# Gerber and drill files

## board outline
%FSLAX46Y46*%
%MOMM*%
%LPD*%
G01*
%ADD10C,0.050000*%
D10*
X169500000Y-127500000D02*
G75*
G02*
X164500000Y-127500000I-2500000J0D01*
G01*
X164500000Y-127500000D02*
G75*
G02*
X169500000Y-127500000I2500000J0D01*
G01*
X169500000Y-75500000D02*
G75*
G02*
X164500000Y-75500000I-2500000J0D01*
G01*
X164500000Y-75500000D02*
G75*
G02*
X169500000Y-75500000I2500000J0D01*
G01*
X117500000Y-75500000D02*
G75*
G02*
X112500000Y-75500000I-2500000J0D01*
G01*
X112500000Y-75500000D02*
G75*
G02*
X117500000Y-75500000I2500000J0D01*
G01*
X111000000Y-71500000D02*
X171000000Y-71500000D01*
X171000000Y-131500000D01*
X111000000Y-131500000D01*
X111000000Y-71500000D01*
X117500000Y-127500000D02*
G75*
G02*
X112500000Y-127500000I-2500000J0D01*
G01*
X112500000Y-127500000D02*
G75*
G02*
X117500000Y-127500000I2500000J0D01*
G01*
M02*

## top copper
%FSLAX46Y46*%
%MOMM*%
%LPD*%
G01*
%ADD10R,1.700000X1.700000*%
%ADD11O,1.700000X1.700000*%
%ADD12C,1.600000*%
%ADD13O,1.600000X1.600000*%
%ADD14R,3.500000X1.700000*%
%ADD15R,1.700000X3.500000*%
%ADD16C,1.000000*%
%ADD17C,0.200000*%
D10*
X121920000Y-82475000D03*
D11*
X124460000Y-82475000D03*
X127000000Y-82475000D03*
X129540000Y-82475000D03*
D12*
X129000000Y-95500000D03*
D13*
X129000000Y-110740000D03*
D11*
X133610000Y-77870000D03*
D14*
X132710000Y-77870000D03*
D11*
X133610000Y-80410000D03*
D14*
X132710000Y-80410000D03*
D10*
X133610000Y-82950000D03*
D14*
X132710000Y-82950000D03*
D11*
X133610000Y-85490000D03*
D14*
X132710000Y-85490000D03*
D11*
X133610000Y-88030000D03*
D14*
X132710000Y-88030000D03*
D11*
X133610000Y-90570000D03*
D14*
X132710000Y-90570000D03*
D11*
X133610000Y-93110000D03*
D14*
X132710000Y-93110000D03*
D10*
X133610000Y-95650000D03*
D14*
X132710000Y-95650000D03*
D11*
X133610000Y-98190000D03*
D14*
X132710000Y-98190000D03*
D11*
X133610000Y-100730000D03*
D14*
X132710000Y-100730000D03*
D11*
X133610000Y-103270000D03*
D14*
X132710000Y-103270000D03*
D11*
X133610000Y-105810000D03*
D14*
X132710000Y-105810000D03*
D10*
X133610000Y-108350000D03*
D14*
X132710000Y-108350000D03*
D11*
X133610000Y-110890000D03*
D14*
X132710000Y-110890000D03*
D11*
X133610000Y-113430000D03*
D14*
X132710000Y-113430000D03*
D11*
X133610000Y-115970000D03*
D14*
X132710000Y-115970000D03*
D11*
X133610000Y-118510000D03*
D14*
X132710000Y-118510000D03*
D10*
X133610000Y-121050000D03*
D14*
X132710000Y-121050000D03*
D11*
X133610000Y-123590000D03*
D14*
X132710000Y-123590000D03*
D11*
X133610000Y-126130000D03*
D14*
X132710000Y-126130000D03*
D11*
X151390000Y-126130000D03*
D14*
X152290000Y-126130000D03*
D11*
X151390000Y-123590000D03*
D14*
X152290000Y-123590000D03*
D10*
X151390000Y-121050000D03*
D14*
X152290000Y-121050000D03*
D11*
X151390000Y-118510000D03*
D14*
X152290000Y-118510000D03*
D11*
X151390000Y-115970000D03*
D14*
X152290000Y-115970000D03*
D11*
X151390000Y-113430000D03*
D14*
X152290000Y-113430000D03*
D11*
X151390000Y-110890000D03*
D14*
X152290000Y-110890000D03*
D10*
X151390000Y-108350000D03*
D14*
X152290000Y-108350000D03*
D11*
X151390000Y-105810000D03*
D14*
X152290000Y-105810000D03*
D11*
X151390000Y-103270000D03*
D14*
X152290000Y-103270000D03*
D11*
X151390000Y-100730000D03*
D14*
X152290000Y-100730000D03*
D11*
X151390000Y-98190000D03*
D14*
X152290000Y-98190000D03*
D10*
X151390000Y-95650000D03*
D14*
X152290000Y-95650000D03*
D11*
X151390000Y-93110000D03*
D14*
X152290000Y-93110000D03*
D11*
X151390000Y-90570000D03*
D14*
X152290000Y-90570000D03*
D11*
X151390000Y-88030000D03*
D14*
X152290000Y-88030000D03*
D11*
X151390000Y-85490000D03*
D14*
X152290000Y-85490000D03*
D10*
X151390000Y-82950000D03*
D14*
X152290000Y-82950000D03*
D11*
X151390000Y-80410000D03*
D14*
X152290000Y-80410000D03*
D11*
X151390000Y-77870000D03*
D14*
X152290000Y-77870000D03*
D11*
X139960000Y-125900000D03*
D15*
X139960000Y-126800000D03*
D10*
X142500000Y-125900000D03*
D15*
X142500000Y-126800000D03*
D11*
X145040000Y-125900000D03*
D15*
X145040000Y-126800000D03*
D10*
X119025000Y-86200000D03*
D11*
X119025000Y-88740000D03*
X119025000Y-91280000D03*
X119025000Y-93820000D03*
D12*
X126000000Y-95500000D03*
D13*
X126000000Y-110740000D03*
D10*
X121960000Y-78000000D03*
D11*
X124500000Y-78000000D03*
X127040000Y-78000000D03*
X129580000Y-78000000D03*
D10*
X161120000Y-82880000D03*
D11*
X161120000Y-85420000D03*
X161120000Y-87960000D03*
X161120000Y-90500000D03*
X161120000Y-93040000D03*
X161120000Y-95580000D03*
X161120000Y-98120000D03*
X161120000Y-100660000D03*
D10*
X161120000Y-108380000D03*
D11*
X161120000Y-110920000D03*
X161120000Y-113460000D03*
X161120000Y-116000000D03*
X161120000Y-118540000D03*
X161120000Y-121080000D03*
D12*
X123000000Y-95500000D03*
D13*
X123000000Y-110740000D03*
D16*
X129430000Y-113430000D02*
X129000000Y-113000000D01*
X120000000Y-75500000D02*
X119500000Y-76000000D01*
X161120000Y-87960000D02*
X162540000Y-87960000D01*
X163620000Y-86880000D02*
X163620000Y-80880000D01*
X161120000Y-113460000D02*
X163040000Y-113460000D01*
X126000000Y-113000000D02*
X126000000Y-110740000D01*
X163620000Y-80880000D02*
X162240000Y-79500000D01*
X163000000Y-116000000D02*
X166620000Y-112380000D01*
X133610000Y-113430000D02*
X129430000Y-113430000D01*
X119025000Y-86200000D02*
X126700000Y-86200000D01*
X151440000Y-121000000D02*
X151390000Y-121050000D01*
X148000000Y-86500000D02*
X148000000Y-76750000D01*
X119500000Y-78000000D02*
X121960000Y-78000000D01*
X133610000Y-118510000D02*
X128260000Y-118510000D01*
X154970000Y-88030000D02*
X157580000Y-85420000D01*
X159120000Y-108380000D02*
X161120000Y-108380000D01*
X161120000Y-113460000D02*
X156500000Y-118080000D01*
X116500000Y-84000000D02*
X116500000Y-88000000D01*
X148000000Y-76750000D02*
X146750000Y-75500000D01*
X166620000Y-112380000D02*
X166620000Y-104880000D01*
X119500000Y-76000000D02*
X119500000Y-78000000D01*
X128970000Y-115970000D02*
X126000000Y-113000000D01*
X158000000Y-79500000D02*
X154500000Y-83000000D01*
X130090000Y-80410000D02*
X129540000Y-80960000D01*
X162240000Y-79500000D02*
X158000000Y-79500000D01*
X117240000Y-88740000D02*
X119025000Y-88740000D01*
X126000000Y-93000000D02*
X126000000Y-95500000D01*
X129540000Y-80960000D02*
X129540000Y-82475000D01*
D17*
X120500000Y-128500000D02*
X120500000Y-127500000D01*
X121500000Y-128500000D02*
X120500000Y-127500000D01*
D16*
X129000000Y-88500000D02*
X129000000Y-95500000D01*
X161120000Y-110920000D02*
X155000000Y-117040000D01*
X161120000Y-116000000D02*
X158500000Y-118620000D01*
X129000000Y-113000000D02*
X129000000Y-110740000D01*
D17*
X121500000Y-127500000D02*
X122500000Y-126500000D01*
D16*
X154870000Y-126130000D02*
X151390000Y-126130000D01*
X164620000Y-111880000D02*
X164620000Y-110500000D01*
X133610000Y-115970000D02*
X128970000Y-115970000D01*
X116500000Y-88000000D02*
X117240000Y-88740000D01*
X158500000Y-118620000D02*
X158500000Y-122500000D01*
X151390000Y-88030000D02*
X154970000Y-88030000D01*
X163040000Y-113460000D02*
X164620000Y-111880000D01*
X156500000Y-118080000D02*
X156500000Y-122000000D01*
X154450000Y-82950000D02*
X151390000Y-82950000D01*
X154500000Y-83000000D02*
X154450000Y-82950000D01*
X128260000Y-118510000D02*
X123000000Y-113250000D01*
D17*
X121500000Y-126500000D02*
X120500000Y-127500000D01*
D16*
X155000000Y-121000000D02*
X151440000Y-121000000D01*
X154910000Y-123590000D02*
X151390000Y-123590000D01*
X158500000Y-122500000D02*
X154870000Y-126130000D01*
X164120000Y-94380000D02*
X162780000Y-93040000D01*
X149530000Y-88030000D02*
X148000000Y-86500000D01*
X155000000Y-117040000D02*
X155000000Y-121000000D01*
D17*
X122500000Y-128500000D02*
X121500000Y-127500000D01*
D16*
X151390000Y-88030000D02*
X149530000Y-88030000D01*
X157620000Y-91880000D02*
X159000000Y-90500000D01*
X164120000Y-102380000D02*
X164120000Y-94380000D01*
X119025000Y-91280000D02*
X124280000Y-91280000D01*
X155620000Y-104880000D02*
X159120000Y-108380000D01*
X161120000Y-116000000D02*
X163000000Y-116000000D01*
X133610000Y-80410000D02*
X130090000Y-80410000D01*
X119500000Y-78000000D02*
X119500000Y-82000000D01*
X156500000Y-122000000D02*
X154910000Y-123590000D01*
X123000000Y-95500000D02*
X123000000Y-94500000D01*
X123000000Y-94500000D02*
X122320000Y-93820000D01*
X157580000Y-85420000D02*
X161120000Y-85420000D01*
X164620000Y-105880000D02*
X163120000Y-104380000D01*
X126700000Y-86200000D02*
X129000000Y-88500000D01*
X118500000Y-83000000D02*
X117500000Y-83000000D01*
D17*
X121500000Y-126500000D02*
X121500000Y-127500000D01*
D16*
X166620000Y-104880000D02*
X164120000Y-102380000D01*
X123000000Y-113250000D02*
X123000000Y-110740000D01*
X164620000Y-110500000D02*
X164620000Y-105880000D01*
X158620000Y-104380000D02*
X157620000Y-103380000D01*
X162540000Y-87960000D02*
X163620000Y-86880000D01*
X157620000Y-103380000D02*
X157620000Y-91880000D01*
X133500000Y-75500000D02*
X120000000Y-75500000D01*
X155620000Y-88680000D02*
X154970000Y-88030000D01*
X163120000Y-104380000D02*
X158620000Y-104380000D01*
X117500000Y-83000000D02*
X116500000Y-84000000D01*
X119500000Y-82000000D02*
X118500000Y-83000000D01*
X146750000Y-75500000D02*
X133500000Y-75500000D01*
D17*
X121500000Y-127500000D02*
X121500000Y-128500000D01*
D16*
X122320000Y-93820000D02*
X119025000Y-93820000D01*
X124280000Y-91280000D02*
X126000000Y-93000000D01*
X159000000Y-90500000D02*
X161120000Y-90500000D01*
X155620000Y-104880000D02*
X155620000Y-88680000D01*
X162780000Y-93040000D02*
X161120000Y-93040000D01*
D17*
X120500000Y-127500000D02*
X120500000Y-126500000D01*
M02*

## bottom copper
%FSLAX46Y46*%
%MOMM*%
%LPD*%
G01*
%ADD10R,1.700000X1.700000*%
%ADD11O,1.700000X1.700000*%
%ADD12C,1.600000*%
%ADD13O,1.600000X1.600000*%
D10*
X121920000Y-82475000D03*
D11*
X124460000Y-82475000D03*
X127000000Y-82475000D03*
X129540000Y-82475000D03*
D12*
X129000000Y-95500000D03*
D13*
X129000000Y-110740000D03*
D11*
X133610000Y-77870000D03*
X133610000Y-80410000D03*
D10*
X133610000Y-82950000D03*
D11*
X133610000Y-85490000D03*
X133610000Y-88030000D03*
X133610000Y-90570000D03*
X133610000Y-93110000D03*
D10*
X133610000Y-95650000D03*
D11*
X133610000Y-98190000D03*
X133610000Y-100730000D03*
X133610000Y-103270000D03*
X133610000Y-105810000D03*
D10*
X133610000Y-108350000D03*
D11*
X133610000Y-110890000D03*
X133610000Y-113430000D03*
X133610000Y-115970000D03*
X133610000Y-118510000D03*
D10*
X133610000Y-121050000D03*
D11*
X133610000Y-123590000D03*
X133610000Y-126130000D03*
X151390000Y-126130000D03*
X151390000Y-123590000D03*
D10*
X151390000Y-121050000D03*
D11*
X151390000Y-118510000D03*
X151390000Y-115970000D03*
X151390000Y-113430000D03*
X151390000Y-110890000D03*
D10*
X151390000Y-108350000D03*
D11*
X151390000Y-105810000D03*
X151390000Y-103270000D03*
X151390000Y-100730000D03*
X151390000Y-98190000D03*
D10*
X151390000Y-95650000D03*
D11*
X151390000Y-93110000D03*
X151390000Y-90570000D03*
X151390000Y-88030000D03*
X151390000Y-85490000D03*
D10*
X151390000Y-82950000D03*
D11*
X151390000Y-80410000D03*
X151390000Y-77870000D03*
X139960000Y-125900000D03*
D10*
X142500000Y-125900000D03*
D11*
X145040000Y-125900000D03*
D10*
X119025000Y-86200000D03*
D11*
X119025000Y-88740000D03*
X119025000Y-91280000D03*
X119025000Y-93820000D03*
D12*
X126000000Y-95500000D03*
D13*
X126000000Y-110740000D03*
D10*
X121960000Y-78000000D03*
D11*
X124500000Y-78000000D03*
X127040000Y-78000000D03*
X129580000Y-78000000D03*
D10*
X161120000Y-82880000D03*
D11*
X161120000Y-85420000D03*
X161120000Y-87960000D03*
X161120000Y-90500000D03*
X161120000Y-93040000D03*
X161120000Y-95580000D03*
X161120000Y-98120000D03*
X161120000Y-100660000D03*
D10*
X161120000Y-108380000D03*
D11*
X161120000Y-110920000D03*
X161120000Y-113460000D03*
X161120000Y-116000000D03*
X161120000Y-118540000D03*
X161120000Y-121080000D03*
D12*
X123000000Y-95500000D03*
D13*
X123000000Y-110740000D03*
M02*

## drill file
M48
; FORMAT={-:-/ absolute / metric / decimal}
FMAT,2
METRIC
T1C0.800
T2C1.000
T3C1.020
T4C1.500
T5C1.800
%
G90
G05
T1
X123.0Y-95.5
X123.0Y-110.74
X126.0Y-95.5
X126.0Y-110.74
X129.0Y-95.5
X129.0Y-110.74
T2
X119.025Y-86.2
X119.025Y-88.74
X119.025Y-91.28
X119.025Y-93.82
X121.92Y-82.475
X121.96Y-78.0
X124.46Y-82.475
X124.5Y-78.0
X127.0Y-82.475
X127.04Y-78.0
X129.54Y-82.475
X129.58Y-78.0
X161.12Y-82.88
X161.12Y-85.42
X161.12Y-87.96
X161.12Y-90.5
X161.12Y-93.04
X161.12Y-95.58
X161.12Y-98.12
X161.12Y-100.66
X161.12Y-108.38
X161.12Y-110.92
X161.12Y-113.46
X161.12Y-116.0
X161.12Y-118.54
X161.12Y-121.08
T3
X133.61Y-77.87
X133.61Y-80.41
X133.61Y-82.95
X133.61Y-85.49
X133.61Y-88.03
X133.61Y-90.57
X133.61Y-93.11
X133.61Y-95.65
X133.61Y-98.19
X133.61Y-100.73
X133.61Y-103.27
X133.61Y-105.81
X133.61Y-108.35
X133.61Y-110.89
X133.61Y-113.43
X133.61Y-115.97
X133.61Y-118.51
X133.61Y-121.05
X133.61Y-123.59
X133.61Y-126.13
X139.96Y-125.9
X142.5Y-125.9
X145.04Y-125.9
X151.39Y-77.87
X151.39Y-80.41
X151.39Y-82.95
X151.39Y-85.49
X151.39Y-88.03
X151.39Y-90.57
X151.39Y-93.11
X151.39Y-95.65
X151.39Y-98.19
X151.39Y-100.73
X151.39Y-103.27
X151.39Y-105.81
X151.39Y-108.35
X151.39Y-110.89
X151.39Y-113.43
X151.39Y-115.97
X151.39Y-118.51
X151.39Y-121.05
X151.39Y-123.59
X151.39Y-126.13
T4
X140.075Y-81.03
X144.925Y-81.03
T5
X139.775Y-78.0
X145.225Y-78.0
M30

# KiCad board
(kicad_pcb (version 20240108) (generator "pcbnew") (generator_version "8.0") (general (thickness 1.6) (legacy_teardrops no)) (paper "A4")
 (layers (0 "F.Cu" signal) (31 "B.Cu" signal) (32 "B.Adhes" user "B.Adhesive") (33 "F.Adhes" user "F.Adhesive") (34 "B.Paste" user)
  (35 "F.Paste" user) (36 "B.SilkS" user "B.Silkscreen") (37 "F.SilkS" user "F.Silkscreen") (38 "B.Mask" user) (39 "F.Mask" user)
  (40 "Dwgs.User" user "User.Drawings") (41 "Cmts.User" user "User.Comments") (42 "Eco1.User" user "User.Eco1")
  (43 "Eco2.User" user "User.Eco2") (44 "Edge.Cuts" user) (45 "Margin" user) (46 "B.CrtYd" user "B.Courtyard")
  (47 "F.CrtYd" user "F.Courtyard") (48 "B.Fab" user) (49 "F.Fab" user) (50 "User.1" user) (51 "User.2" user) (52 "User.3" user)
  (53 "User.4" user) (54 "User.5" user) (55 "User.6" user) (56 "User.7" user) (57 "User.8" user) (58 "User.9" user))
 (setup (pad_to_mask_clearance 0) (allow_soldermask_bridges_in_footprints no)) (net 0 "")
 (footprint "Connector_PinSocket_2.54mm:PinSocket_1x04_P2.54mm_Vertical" (layer "F.Cu") (at 121.92 82.475 90)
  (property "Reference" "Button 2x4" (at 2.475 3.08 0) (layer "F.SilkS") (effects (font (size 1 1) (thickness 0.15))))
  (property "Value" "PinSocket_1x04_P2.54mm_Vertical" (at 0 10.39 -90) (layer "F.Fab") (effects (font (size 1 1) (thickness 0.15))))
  (pad "1" thru_hole rect (at 0 0 90) (size 1.7 1.7) (drill 1) (layers "*.Cu" "*.Mask") (remove_unused_layers no))
  (pad "2" thru_hole oval (at 0 2.54 90) (size 1.7 1.7) (drill 1) (layers "*.Cu" "*.Mask") (remove_unused_layers no))
  (pad "3" thru_hole oval (at 0 5.08 90) (size 1.7 1.7) (drill 1) (layers "*.Cu" "*.Mask") (remove_unused_layers no))
  (pad "4" thru_hole oval (at 0 7.62 90) (size 1.7 1.7) (drill 1) (layers "*.Cu" "*.Mask") (remove_unused_layers no)))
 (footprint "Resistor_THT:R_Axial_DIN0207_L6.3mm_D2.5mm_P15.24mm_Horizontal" (layer "F.Cu") (at 129 95.5 -90)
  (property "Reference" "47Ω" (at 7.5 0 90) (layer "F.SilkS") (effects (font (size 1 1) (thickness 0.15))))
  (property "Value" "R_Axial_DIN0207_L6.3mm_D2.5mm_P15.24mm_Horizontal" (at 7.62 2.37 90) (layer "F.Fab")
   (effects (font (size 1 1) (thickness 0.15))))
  (pad "1" thru_hole circle (at 0 0 270) (size 1.6 1.6) (drill 0.8) (layers "*.Cu" "*.Mask") (remove_unused_layers no))
  (pad "2" thru_hole oval (at 15.24 0 270) (size 1.6 1.6) (drill 0.8) (layers "*.Cu" "*.Mask") (remove_unused_layers no)))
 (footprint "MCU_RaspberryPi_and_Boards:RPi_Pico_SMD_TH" (layer "F.Cu") (at 142.5 102)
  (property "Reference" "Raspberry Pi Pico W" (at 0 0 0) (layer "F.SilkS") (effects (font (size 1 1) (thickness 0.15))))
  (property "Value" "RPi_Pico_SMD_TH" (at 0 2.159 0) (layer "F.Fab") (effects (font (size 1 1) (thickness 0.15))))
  (pad "" np_thru_hole oval (at -2.725 -24) (size 1.8 1.8) (drill 1.8) (layers "*.Cu" "*.Mask"))
  (pad "" np_thru_hole oval (at -2.425 -20.97) (size 1.5 1.5) (drill 1.5) (layers "*.Cu" "*.Mask"))
  (pad "" np_thru_hole oval (at 2.425 -20.97) (size 1.5 1.5) (drill 1.5) (layers "*.Cu" "*.Mask"))
  (pad "" np_thru_hole oval (at 2.725 -24) (size 1.8 1.8) (drill 1.8) (layers "*.Cu" "*.Mask"))
  (pad "1" thru_hole oval (at -8.89 -24.13) (size 1.7 1.7) (drill 1.02) (layers "*.Cu" "*.Mask") (remove_unused_layers no))
  (pad "1" smd rect (at -8.89 -24.13) (size 3.5 1.7) (drill (offset -0.9 0)) (layers "F.Cu" "F.Mask"))
  (pad "2" thru_hole oval (at -8.89 -21.59) (size 1.7 1.7) (drill 1.02) (layers "*.Cu" "*.Mask") (remove_unused_layers no))
  (pad "2" smd rect (at -8.89 -21.59) (size 3.5 1.7) (drill (offset -0.9 0)) (layers "F.Cu" "F.Mask"))
  (pad "3" thru_hole rect (at -8.89 -19.05) (size 1.7 1.7) (drill 1.02) (layers "*.Cu" "*.Mask") (remove_unused_layers no))
  (pad "3" smd rect (at -8.89 -19.05) (size 3.5 1.7) (drill (offset -0.9 0)) (layers "F.Cu" "F.Mask"))
  (pad "4" thru_hole oval (at -8.89 -16.51) (size 1.7 1.7) (drill 1.02) (layers "*.Cu" "*.Mask") (remove_unused_layers no))
  (pad "4" smd rect (at -8.89 -16.51) (size 3.5 1.7) (drill (offset -0.9 0)) (layers "F.Cu" "F.Mask"))
  (pad "5" thru_hole oval (at -8.89 -13.97) (size 1.7 1.7) (drill 1.02) (layers "*.Cu" "*.Mask") (remove_unused_layers no))
  (pad "5" smd rect (at -8.89 -13.97) (size 3.5 1.7) (drill (offset -0.9 0)) (layers "F.Cu" "F.Mask"))
  (pad "6" thru_hole oval (at -8.89 -11.43) (size 1.7 1.7) (drill 1.02) (layers "*.Cu" "*.Mask") (remove_unused_layers no))
  (pad "6" smd rect (at -8.89 -11.43) (size 3.5 1.7) (drill (offset -0.9 0)) (layers "F.Cu" "F.Mask"))
  (pad "7" thru_hole oval (at -8.89 -8.89) (size 1.7 1.7) (drill 1.02) (layers "*.Cu" "*.Mask") (remove_unused_layers no))
  (pad "7" smd rect (at -8.89 -8.89) (size 3.5 1.7) (drill (offset -0.9 0)) (layers "F.Cu" "F.Mask"))
  (pad "8" thru_hole rect (at -8.89 -6.35) (size 1.7 1.7) (drill 1.02) (layers "*.Cu" "*.Mask") (remove_unused_layers no))
  (pad "8" smd rect (at -8.89 -6.35) (size 3.5 1.7) (drill (offset -0.9 0)) (layers "F.Cu" "F.Mask"))
  (pad "9" thru_hole oval (at -8.89 -3.81) (size 1.7 1.7) (drill 1.02) (layers "*.Cu" "*.Mask") (remove_unused_layers no))
  (pad "9" smd rect (at -8.89 -3.81) (size 3.5 1.7) (drill (offset -0.9 0)) (layers "F.Cu" "F.Mask"))
  (pad "10" thru_hole oval (at -8.89 -1.27) (size 1.7 1.7) (drill 1.02) (layers "*.Cu" "*.Mask") (remove_unused_layers no))
  (pad "10" smd rect (at -8.89 -1.27) (size 3.5 1.7) (drill (offset -0.9 0)) (layers "F.Cu" "F.Mask"))
  (pad "11" thru_hole oval (at -8.89 1.27) (size 1.7 1.7) (drill 1.02) (layers "*.Cu" "*.Mask") (remove_unused_layers no))
  (pad "11" smd rect (at -8.89 1.27) (size 3.5 1.7) (drill (offset -0.9 0)) (layers "F.Cu" "F.Mask"))
  (pad "12" thru_hole oval (at -8.89 3.81) (size 1.7 1.7) (drill 1.02) (layers "*.Cu" "*.Mask") (remove_unused_layers no))
  (pad "12" smd rect (at -8.89 3.81) (size 3.5 1.7) (drill (offset -0.9 0)) (layers "F.Cu" "F.Mask"))
  (pad "13" thru_hole rect (at -8.89 6.35) (size 1.7 1.7) (drill 1.02) (layers "*.Cu" "*.Mask") (remove_unused_layers no))
  (pad "13" smd rect (at -8.89 6.35) (size 3.5 1.7) (drill (offset -0.9 0)) (layers "F.Cu" "F.Mask"))
  (pad "14" thru_hole oval (at -8.89 8.89) (size 1.7 1.7) (drill 1.02) (layers "*.Cu" "*.Mask") (remove_unused_layers no))
  (pad "14" smd rect (at -8.89 8.89) (size 3.5 1.7) (drill (offset -0.9 0)) (layers "F.Cu" "F.Mask"))
  (pad "15" thru_hole oval (at -8.89 11.43) (size 1.7 1.7) (drill 1.02) (layers "*.Cu" "*.Mask") (remove_unused_layers no))
  (pad "15" smd rect (at -8.89 11.43) (size 3.5 1.7) (drill (offset -0.9 0)) (layers "F.Cu" "F.Mask"))
  (pad "16" thru_hole oval (at -8.89 13.97) (size 1.7 1.7) (drill 1.02) (layers "*.Cu" "*.Mask") (remove_unused_layers no))
  (pad "16" smd rect (at -8.89 13.97) (size 3.5 1.7) (drill (offset -0.9 0)) (layers "F.Cu" "F.Mask"))
  (pad "17" thru_hole oval (at -8.89 16.51) (size 1.7 1.7) (drill 1.02) (layers "*.Cu" "*.Mask") (remove_unused_layers no))
  (pad "17" smd rect (at -8.89 16.51) (size 3.5 1.7) (drill (offset -0.9 0)) (layers "F.Cu" "F.Mask"))
  (pad "18" thru_hole rect (at -8.89 19.05) (size 1.7 1.7) (drill 1.02) (layers "*.Cu" "*.Mask") (remove_unused_layers no))
  (pad "18" smd rect (at -8.89 19.05) (size 3.5 1.7) (drill (offset -0.9 0)) (layers "F.Cu" "F.Mask"))
  (pad "19" thru_hole oval (at -8.89 21.59) (size 1.7 1.7) (drill 1.02) (layers "*.Cu" "*.Mask") (remove_unused_layers no))
  (pad "19" smd rect (at -8.89 21.59) (size 3.5 1.7) (drill (offset -0.9 0)) (layers "F.Cu" "F.Mask"))
  (pad "20" thru_hole oval (at -8.89 24.13) (size 1.7 1.7) (drill 1.02) (layers "*.Cu" "*.Mask") (remove_unused_layers no))
  (pad "20" smd rect (at -8.89 24.13) (size 3.5 1.7) (drill (offset -0.9 0)) (layers "F.Cu" "F.Mask"))
  (pad "21" thru_hole oval (at 8.89 24.13) (size 1.7 1.7) (drill 1.02) (layers "*.Cu" "*.Mask") (remove_unused_layers no))
  (pad "21" smd rect (at 8.89 24.13) (size 3.5 1.7) (drill (offset 0.9 0)) (layers "F.Cu" "F.Mask"))
  (pad "22" thru_hole oval (at 8.89 21.59) (size 1.7 1.7) (drill 1.02) (layers "*.Cu" "*.Mask") (remove_unused_layers no))
  (pad "22" smd rect (at 8.89 21.59) (size 3.5 1.7) (drill (offset 0.9 0)) (layers "F.Cu" "F.Mask"))
  (pad "23" thru_hole rect (at 8.89 19.05) (size 1.7 1.7) (drill 1.02) (layers "*.Cu" "*.Mask") (remove_unused_layers no))
  (pad "23" smd rect (at 8.89 19.05) (size 3.5 1.7) (drill (offset 0.9 0)) (layers "F.Cu" "F.Mask"))
  (pad "24" thru_hole oval (at 8.89 16.51) (size 1.7 1.7) (drill 1.02) (layers "*.Cu" "*.Mask") (remove_unused_layers no))
  (pad "24" smd rect (at 8.89 16.51) (size 3.5 1.7) (drill (offset 0.9 0)) (layers "F.Cu" "F.Mask"))
  (pad "25" thru_hole oval (at 8.89 13.97) (size 1.7 1.7) (drill 1.02) (layers "*.Cu" "*.Mask") (remove_unused_layers no))
  (pad "25" smd rect (at 8.89 13.97) (size 3.5 1.7) (drill (offset 0.9 0)) (layers "F.Cu" "F.Mask"))
  (pad "26" thru_hole oval (at 8.89 11.43) (size 1.7 1.7) (drill 1.02) (layers "*.Cu" "*.Mask") (remove_unused_layers no))
  (pad "26" smd rect (at 8.89 11.43) (size 3.5 1.7) (drill (offset 0.9 0)) (layers "F.Cu" "F.Mask"))
  (pad "27" thru_hole oval (at 8.89 8.89) (size 1.7 1.7) (drill 1.02) (layers "*.Cu" "*.Mask") (remove_unused_layers no))
  (pad "27" smd rect (at 8.89 8.89) (size 3.5 1.7) (drill (offset 0.9 0)) (layers "F.Cu" "F.Mask"))
  (pad "28" thru_hole rect (at 8.89 6.35) (size 1.7 1.7) (drill 1.02) (layers "*.Cu" "*.Mask") (remove_unused_layers no))
  (pad "28" smd rect (at 8.89 6.35) (size 3.5 1.7) (drill (offset 0.9 0)) (layers "F.Cu" "F.Mask"))
  (pad "29" thru_hole oval (at 8.89 3.81) (size 1.7 1.7) (drill 1.02) (layers "*.Cu" "*.Mask") (remove_unused_layers no))
  (pad "29" smd rect (at 8.89 3.81) (size 3.5 1.7) (drill (offset 0.9 0)) (layers "F.Cu" "F.Mask"))
  (pad "30" thru_hole oval (at 8.89 1.27) (size 1.7 1.7) (drill 1.02) (layers "*.Cu" "*.Mask") (remove_unused_layers no))
  (pad "30" smd rect (at 8.89 1.27) (size 3.5 1.7) (drill (offset 0.9 0)) (layers "F.Cu" "F.Mask"))
  (pad "31" thru_hole oval (at 8.89 -1.27) (size 1.7 1.7) (drill 1.02) (layers "*.Cu" "*.Mask") (remove_unused_layers no))
  (pad "31" smd rect (at 8.89 -1.27) (size 3.5 1.7) (drill (offset 0.9 0)) (layers "F.Cu" "F.Mask"))
  (pad "32" thru_hole oval (at 8.89 -3.81) (size 1.7 1.7) (drill 1.02) (layers "*.Cu" "*.Mask") (remove_unused_layers no))
  (pad "32" smd rect (at 8.89 -3.81) (size 3.5 1.7) (drill (offset 0.9 0)) (layers "F.Cu" "F.Mask"))
  (pad "33" thru_hole rect (at 8.89 -6.35) (size 1.7 1.7) (drill 1.02) (layers "*.Cu" "*.Mask") (remove_unused_layers no))
  (pad "33" smd rect (at 8.89 -6.35) (size 3.5 1.7) (drill (offset 0.9 0)) (layers "F.Cu" "F.Mask"))
  (pad "34" thru_hole oval (at 8.89 -8.89) (size 1.7 1.7) (drill 1.02) (layers "*.Cu" "*.Mask") (remove_unused_layers no))
  (pad "34" smd rect (at 8.89 -8.89) (size 3.5 1.7) (drill (offset 0.9 0)) (layers "F.Cu" "F.Mask"))
  (pad "35" thru_hole oval (at 8.89 -11.43) (size 1.7 1.7) (drill 1.02) (layers "*.Cu" "*.Mask") (remove_unused_layers no))
  (pad "35" smd rect (at 8.89 -11.43) (size 3.5 1.7) (drill (offset 0.9 0)) (layers "F.Cu" "F.Mask"))
  (pad "36" thru_hole oval (at 8.89 -13.97) (size 1.7 1.7) (drill 1.02) (layers "*.Cu" "*.Mask") (remove_unused_layers no))
  (pad "36" smd rect (at 8.89 -13.97) (size 3.5 1.7) (drill (offset 0.9 0)) (layers "F.Cu" "F.Mask"))
  (pad "37" thru_hole oval (at 8.89 -16.51) (size 1.7 1.7) (drill 1.02) (layers "*.Cu" "*.Mask") (remove_unused_layers no))
  (pad "37" smd rect (at 8.89 -16.51) (size 3.5 1.7) (drill (offset 0.9 0)) (layers "F.Cu" "F.Mask"))
  (pad "38" thru_hole rect (at 8.89 -19.05) (size 1.7 1.7) (drill 1.02) (layers "*.Cu" "*.Mask") (remove_unused_layers no))
  (pad "38" smd rect (at 8.89 -19.05) (size 3.5 1.7) (drill (offset 0.9 0)) (layers "F.Cu" "F.Mask"))
  (pad "39" thru_hole oval (at 8.89 -21.59) (size 1.7 1.7) (drill 1.02) (layers "*.Cu" "*.Mask") (remove_unused_layers no))
  (pad "39" smd rect (at 8.89 -21.59) (size 3.5 1.7) (drill (offset 0.9 0)) (layers "F.Cu" "F.Mask"))
  (pad "40" thru_hole oval (at 8.89 -24.13) (size 1.7 1.7) (drill 1.02) (layers "*.Cu" "*.Mask") (remove_unused_layers no))
  (pad "40" smd rect (at 8.89 -24.13) (size 3.5 1.7) (drill (offset 0.9 0)) (layers "F.Cu" "F.Mask"))
  (pad "41" thru_hole oval (at -2.54 23.9) (size 1.7 1.7) (drill 1.02) (layers "*.Cu" "*.Mask") (remove_unused_layers no))
  (pad "41" smd rect (at -2.54 23.9 90) (size 3.5 1.7) (drill (offset -0.9 0)) (layers "F.Cu" "F.Mask"))
  (pad "42" thru_hole rect (at 0 23.9) (size 1.7 1.7) (drill 1.02) (layers "*.Cu" "*.Mask") (remove_unused_layers no))
  (pad "42" smd rect (at 0 23.9 90) (size 3.5 1.7) (drill (offset -0.9 0)) (layers "F.Cu" "F.Mask"))
  (pad "43" thru_hole oval (at 2.54 23.9) (size 1.7 1.7) (drill 1.02) (layers "*.Cu" "*.Mask") (remove_unused_layers no))
  (pad "43" smd rect (at 2.54 23.9 90) (size 3.5 1.7) (drill (offset -0.9 0)) (layers "F.Cu" "F.Mask")))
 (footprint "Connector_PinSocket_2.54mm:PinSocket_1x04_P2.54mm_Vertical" (layer "F.Cu") (at 119.025 86.2)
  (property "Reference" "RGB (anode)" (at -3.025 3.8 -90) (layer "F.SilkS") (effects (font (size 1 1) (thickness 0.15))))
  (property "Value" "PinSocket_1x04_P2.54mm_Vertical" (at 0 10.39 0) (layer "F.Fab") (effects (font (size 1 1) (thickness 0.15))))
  (pad "1" thru_hole rect (at 0 0) (size 1.7 1.7) (drill 1) (layers "*.Cu" "*.Mask") (remove_unused_layers no))
  (pad "2" thru_hole oval (at 0 2.54) (size 1.7 1.7) (drill 1) (layers "*.Cu" "*.Mask") (remove_unused_layers no))
  (pad "3" thru_hole oval (at 0 5.08) (size 1.7 1.7) (drill 1) (layers "*.Cu" "*.Mask") (remove_unused_layers no))
  (pad "4" thru_hole oval (at 0 7.62) (size 1.7 1.7) (drill 1) (layers "*.Cu" "*.Mask") (remove_unused_layers no)))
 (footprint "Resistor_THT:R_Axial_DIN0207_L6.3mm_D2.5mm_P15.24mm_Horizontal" (layer "F.Cu") (at 126 95.5 -90)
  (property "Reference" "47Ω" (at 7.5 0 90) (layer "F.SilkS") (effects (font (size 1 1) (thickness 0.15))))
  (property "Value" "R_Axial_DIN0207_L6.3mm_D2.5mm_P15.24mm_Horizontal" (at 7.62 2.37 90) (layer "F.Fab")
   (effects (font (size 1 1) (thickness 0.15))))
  (pad "1" thru_hole circle (at 0 0 270) (size 1.6 1.6) (drill 0.8) (layers "*.Cu" "*.Mask") (remove_unused_layers no))
  (pad "2" thru_hole oval (at 15.24 0 270) (size 1.6 1.6) (drill 0.8) (layers "*.Cu" "*.Mask") (remove_unused_layers no)))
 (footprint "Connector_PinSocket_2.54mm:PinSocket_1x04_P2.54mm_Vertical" (layer "F.Cu") (at 121.96 78 90)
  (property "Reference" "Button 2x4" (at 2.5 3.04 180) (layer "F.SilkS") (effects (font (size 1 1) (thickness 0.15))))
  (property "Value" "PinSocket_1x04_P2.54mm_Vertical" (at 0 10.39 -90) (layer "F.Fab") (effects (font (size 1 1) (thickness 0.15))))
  (pad "1" thru_hole rect (at 0 0 90) (size 1.7 1.7) (drill 1) (layers "*.Cu" "*.Mask") (remove_unused_layers no))
  (pad "2" thru_hole oval (at 0 2.54 90) (size 1.7 1.7) (drill 1) (layers "*.Cu" "*.Mask") (remove_unused_layers no))
  (pad "3" thru_hole oval (at 0 5.08 90) (size 1.7 1.7) (drill 1) (layers "*.Cu" "*.Mask") (remove_unused_layers no))
  (pad "4" thru_hole oval (at 0 7.62 90) (size 1.7 1.7) (drill 1) (layers "*.Cu" "*.Mask") (remove_unused_layers no)))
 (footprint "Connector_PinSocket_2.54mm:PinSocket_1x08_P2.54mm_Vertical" (layer "F.Cu") (at 161.12 82.88)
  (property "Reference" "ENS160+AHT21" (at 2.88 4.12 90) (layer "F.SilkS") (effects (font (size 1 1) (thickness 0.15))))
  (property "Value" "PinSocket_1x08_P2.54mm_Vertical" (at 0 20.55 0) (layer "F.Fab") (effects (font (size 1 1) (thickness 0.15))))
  (pad "1" thru_hole rect (at 0 0) (size 1.7 1.7) (drill 1) (layers "*.Cu" "*.Mask") (remove_unused_layers no))
  (pad "2" thru_hole oval (at 0 2.54) (size 1.7 1.7) (drill 1) (layers "*.Cu" "*.Mask") (remove_unused_layers no))
  (pad "3" thru_hole oval (at 0 5.08) (size 1.7 1.7) (drill 1) (layers "*.Cu" "*.Mask") (remove_unused_layers no))
  (pad "4" thru_hole oval (at 0 7.62) (size 1.7 1.7) (drill 1) (layers "*.Cu" "*.Mask") (remove_unused_layers no))
  (pad "5" thru_hole oval (at 0 10.16) (size 1.7 1.7) (drill 1) (layers "*.Cu" "*.Mask") (remove_unused_layers no))
  (pad "6" thru_hole oval (at 0 12.7) (size 1.7 1.7) (drill 1) (layers "*.Cu" "*.Mask") (remove_unused_layers no))
  (pad "7" thru_hole oval (at 0 15.24) (size 1.7 1.7) (drill 1) (layers "*.Cu" "*.Mask") (remove_unused_layers no))
  (pad "8" thru_hole oval (at 0 17.78) (size 1.7 1.7) (drill 1) (layers "*.Cu" "*.Mask") (remove_unused_layers no)))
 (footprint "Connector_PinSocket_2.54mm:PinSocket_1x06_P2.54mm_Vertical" (layer "F.Cu") (at 161.12 108.38)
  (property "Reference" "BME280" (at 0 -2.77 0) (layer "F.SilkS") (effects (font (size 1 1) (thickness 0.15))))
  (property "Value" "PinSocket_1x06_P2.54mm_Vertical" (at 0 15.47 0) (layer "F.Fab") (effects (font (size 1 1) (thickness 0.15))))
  (pad "1" thru_hole rect (at 0 0) (size 1.7 1.7) (drill 1) (layers "*.Cu" "*.Mask") (remove_unused_layers no))
  (pad "2" thru_hole oval (at 0 2.54) (size 1.7 1.7) (drill 1) (layers "*.Cu" "*.Mask") (remove_unused_layers no))
  (pad "3" thru_hole oval (at 0 5.08) (size 1.7 1.7) (drill 1) (layers "*.Cu" "*.Mask") (remove_unused_layers no))
  (pad "4" thru_hole oval (at 0 7.62) (size 1.7 1.7) (drill 1) (layers "*.Cu" "*.Mask") (remove_unused_layers no))
  (pad "5" thru_hole oval (at 0 10.16) (size 1.7 1.7) (drill 1) (layers "*.Cu" "*.Mask") (remove_unused_layers no))
  (pad "6" thru_hole oval (at 0 12.7) (size 1.7 1.7) (drill 1) (layers "*.Cu" "*.Mask") (remove_unused_layers no)))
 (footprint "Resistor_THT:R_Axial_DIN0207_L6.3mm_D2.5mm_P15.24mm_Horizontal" (layer "F.Cu") (at 123 95.5 -90)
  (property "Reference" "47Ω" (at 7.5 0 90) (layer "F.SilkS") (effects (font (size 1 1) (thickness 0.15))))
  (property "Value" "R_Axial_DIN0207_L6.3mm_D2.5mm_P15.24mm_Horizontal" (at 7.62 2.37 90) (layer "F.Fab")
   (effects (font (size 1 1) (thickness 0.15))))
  (pad "1" thru_hole circle (at 0 0 270) (size 1.6 1.6) (drill 0.8) (layers "*.Cu" "*.Mask") (remove_unused_layers no))
  (pad "2" thru_hole oval (at 15.24 0 270) (size 1.6 1.6) (drill 0.8) (layers "*.Cu" "*.Mask") (remove_unused_layers no)))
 (gr_circle (center 167 127.5) (end 165 126) (stroke (width 0.05) (type default)) (fill none) (layer "Edge.Cuts"))
 (gr_circle (center 167 75.5) (end 165.5 77.5) (stroke (width 0.05) (type default)) (fill none) (layer "Edge.Cuts"))
 (gr_circle (center 115 75.5) (end 113.5 73.5) (stroke (width 0.05) (type default)) (fill none) (layer "Edge.Cuts"))
 (gr_rect (start 111 71.5) (end 171 131.5) (stroke (width 0.05) (type default)) (fill none) (layer "Edge.Cuts"))
 (gr_circle (center 115 127.5) (end 117 126) (stroke (width 0.05) (type default)) (fill none) (layer "Edge.Cuts"))
 (segment (start 129.43 113.43) (end 129 113) (width 1) (layer "F.Cu") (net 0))
 (segment (start 120 75.5) (end 119.5 76) (width 1) (layer "F.Cu") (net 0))
 (segment (start 161.12 87.96) (end 162.54 87.96) (width 1) (layer "F.Cu") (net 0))
 (segment (start 163.62 86.88) (end 163.62 80.88) (width 1) (layer "F.Cu") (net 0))
 (segment (start 161.12 113.46) (end 163.04 113.46) (width 1) (layer "F.Cu") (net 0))
 (segment (start 126 113) (end 126 110.74) (width 1) (layer "F.Cu") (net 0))
 (segment (start 163.62 80.88) (end 162.24 79.5) (width 1) (layer "F.Cu") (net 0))
 (segment (start 163 116) (end 166.62 112.38) (width 1) (layer "F.Cu") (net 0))
 (segment (start 133.61 113.43) (end 129.43 113.43) (width 1) (layer "F.Cu") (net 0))
 (segment (start 119.025 86.2) (end 126.7 86.2) (width 1) (layer "F.Cu") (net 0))
 (segment (start 151.44 121) (end 151.39 121.05) (width 1) (layer "F.Cu") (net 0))
 (segment (start 148 86.5) (end 148 76.75) (width 1) (layer "F.Cu") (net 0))
 (segment (start 119.5 78) (end 121.96 78) (width 1) (layer "F.Cu") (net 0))
 (segment (start 133.61 118.51) (end 128.26 118.51) (width 1) (layer "F.Cu") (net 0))
 (segment (start 154.97 88.03) (end 157.58 85.42) (width 1) (layer "F.Cu") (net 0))
 (segment (start 159.12 108.38) (end 161.12 108.38) (width 1) (layer "F.Cu") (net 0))
 (segment (start 161.12 113.46) (end 156.5 118.08) (width 1) (layer "F.Cu") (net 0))
 (segment (start 116.5 84) (end 116.5 88) (width 1) (layer "F.Cu") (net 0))
 (segment (start 148 76.75) (end 146.75 75.5) (width 1) (layer "F.Cu") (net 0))
 (segment (start 166.62 112.38) (end 166.62 104.88) (width 1) (layer "F.Cu") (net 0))
 (segment (start 119.5 76) (end 119.5 78) (width 1) (layer "F.Cu") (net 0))
 (segment (start 128.97 115.97) (end 126 113) (width 1) (layer "F.Cu") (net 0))
 (segment (start 158 79.5) (end 154.5 83) (width 1) (layer "F.Cu") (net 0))
 (segment (start 130.09 80.41) (end 129.54 80.96) (width 1) (layer "F.Cu") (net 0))
 (segment (start 162.24 79.5) (end 158 79.5) (width 1) (layer "F.Cu") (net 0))
 (segment (start 117.24 88.74) (end 119.025 88.74) (width 1) (layer "F.Cu") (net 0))
 (segment (start 126 93) (end 126 95.5) (width 1) (layer "F.Cu") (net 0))
 (segment (start 129.54 80.96) (end 129.54 82.475) (width 1) (layer "F.Cu") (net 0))
 (segment (start 120.5 128.5) (end 120.5 127.5) (width 0.2) (layer "F.Cu") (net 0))
 (segment (start 121.5 128.5) (end 120.5 127.5) (width 0.2) (layer "F.Cu") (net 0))
 (segment (start 129 88.5) (end 129 95.5) (width 1) (layer "F.Cu") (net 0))
 (segment (start 161.12 110.92) (end 155 117.04) (width 1) (layer "F.Cu") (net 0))
 (segment (start 161.12 116) (end 158.5 118.62) (width 1) (layer "F.Cu") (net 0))
 (segment (start 129 113) (end 129 110.74) (width 1) (layer "F.Cu") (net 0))
 (segment (start 121.5 127.5) (end 122.5 126.5) (width 0.2) (layer "F.Cu") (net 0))
 (segment (start 154.87 126.13) (end 151.39 126.13) (width 1) (layer "F.Cu") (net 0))
 (segment (start 164.62 111.88) (end 164.62 110.5) (width 1) (layer "F.Cu") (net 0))
 (segment (start 133.61 115.97) (end 128.97 115.97) (width 1) (layer "F.Cu") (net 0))
 (segment (start 116.5 88) (end 117.24 88.74) (width 1) (layer "F.Cu") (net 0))
 (segment (start 158.5 118.62) (end 158.5 122.5) (width 1) (layer "F.Cu") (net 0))
 (segment (start 151.39 88.03) (end 154.97 88.03) (width 1) (layer "F.Cu") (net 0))
 (segment (start 163.04 113.46) (end 164.62 111.88) (width 1) (layer "F.Cu") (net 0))
 (segment (start 156.5 118.08) (end 156.5 122) (width 1) (layer "F.Cu") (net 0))
 (segment (start 154.45 82.95) (end 151.39 82.95) (width 1) (layer "F.Cu") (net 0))
 (segment (start 154.5 83) (end 154.45 82.95) (width 1) (layer "F.Cu") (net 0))
 (segment (start 128.26 118.51) (end 123 113.25) (width 1) (layer "F.Cu") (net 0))
 (segment (start 121.5 126.5) (end 120.5 127.5) (width 0.2) (layer "F.Cu") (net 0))
 (segment (start 155 121) (end 151.44 121) (width 1) (layer "F.Cu") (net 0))
 (segment (start 154.91 123.59) (end 151.39 123.59) (width 1) (layer "F.Cu") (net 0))
 (segment (start 158.5 122.5) (end 154.87 126.13) (width 1) (layer "F.Cu") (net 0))
 (segment (start 164.12 94.38) (end 162.78 93.04) (width 1) (layer "F.Cu") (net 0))
 (segment (start 149.53 88.03) (end 148 86.5) (width 1) (layer "F.Cu") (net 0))
 (segment (start 155 117.04) (end 155 121) (width 1) (layer "F.Cu") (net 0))
 (segment (start 122.5 128.5) (end 121.5 127.5) (width 0.2) (layer "F.Cu") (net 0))
 (segment (start 151.39 88.03) (end 149.53 88.03) (width 1) (layer "F.Cu") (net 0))
 (segment (start 157.62 91.88) (end 159 90.5) (width 1) (layer "F.Cu") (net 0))
 (segment (start 164.12 102.38) (end 164.12 94.38) (width 1) (layer "F.Cu") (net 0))
 (segment (start 119.025 91.28) (end 124.28 91.28) (width 1) (layer "F.Cu") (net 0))
 (segment (start 155.62 104.88) (end 159.12 108.38) (width 1) (layer "F.Cu") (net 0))
 (segment (start 161.12 116) (end 163 116) (width 1) (layer "F.Cu") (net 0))
 (segment (start 133.61 80.41) (end 130.09 80.41) (width 1) (layer "F.Cu") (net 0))
 (segment (start 119.5 78) (end 119.5 82) (width 1) (layer "F.Cu") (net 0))
 (segment (start 156.5 122) (end 154.91 123.59) (width 1) (layer "F.Cu") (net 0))
 (segment (start 123 95.5) (end 123 94.5) (width 1) (layer "F.Cu") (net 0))
 (segment (start 123 94.5) (end 122.32 93.82) (width 1) (layer "F.Cu") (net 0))
 (segment (start 157.58 85.42) (end 161.12 85.42) (width 1) (layer "F.Cu") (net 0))
 (segment (start 164.62 105.88) (end 163.12 104.38) (width 1) (layer "F.Cu") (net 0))
 (segment (start 126.7 86.2) (end 129 88.5) (width 1) (layer "F.Cu") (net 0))
 (segment (start 118.5 83) (end 117.5 83) (width 1) (layer "F.Cu") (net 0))
 (segment (start 121.5 126.5) (end 121.5 127.5) (width 0.2) (layer "F.Cu") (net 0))
 (segment (start 166.62 104.88) (end 164.12 102.38) (width 1) (layer "F.Cu") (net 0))
 (segment (start 123 113.25) (end 123 110.74) (width 1) (layer "F.Cu") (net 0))
 (segment (start 164.62 110.5) (end 164.62 105.88) (width 1) (layer "F.Cu") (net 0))
 (segment (start 158.62 104.38) (end 157.62 103.38) (width 1) (layer "F.Cu") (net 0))
 (segment (start 162.54 87.96) (end 163.62 86.88) (width 1) (layer "F.Cu") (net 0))
 (segment (start 157.62 103.38) (end 157.62 91.88) (width 1) (layer "F.Cu") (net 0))
 (segment (start 133.5 75.5) (end 120 75.5) (width 1) (layer "F.Cu") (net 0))
 (segment (start 155.62 88.68) (end 154.97 88.03) (width 1) (layer "F.Cu") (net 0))
 (segment (start 163.12 104.38) (end 158.62 104.38) (width 1) (layer "F.Cu") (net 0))
 (segment (start 117.5 83) (end 116.5 84) (width 1) (layer "F.Cu") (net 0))
 (segment (start 119.5 82) (end 118.5 83) (width 1) (layer "F.Cu") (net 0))
 (segment (start 146.75 75.5) (end 133.5 75.5) (width 1) (layer "F.Cu") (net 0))
 (segment (start 121.5 127.5) (end 121.5 128.5) (width 0.2) (layer "F.Cu") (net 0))
 (segment (start 122.32 93.82) (end 119.025 93.82) (width 1) (layer "F.Cu") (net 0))
 (segment (start 124.28 91.28) (end 126 93) (width 1) (layer "F.Cu") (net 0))
 (segment (start 159 90.5) (end 161.12 90.5) (width 1) (layer "F.Cu") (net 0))
 (segment (start 155.62 104.88) (end 155.62 88.68) (width 1) (layer "F.Cu") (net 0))
 (segment (start 162.78 93.04) (end 161.12 93.04) (width 1) (layer "F.Cu") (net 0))
 (segment (start 120.5 127.5) (end 120.5 126.5) (width 0.2) (layer "F.Cu") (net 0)))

